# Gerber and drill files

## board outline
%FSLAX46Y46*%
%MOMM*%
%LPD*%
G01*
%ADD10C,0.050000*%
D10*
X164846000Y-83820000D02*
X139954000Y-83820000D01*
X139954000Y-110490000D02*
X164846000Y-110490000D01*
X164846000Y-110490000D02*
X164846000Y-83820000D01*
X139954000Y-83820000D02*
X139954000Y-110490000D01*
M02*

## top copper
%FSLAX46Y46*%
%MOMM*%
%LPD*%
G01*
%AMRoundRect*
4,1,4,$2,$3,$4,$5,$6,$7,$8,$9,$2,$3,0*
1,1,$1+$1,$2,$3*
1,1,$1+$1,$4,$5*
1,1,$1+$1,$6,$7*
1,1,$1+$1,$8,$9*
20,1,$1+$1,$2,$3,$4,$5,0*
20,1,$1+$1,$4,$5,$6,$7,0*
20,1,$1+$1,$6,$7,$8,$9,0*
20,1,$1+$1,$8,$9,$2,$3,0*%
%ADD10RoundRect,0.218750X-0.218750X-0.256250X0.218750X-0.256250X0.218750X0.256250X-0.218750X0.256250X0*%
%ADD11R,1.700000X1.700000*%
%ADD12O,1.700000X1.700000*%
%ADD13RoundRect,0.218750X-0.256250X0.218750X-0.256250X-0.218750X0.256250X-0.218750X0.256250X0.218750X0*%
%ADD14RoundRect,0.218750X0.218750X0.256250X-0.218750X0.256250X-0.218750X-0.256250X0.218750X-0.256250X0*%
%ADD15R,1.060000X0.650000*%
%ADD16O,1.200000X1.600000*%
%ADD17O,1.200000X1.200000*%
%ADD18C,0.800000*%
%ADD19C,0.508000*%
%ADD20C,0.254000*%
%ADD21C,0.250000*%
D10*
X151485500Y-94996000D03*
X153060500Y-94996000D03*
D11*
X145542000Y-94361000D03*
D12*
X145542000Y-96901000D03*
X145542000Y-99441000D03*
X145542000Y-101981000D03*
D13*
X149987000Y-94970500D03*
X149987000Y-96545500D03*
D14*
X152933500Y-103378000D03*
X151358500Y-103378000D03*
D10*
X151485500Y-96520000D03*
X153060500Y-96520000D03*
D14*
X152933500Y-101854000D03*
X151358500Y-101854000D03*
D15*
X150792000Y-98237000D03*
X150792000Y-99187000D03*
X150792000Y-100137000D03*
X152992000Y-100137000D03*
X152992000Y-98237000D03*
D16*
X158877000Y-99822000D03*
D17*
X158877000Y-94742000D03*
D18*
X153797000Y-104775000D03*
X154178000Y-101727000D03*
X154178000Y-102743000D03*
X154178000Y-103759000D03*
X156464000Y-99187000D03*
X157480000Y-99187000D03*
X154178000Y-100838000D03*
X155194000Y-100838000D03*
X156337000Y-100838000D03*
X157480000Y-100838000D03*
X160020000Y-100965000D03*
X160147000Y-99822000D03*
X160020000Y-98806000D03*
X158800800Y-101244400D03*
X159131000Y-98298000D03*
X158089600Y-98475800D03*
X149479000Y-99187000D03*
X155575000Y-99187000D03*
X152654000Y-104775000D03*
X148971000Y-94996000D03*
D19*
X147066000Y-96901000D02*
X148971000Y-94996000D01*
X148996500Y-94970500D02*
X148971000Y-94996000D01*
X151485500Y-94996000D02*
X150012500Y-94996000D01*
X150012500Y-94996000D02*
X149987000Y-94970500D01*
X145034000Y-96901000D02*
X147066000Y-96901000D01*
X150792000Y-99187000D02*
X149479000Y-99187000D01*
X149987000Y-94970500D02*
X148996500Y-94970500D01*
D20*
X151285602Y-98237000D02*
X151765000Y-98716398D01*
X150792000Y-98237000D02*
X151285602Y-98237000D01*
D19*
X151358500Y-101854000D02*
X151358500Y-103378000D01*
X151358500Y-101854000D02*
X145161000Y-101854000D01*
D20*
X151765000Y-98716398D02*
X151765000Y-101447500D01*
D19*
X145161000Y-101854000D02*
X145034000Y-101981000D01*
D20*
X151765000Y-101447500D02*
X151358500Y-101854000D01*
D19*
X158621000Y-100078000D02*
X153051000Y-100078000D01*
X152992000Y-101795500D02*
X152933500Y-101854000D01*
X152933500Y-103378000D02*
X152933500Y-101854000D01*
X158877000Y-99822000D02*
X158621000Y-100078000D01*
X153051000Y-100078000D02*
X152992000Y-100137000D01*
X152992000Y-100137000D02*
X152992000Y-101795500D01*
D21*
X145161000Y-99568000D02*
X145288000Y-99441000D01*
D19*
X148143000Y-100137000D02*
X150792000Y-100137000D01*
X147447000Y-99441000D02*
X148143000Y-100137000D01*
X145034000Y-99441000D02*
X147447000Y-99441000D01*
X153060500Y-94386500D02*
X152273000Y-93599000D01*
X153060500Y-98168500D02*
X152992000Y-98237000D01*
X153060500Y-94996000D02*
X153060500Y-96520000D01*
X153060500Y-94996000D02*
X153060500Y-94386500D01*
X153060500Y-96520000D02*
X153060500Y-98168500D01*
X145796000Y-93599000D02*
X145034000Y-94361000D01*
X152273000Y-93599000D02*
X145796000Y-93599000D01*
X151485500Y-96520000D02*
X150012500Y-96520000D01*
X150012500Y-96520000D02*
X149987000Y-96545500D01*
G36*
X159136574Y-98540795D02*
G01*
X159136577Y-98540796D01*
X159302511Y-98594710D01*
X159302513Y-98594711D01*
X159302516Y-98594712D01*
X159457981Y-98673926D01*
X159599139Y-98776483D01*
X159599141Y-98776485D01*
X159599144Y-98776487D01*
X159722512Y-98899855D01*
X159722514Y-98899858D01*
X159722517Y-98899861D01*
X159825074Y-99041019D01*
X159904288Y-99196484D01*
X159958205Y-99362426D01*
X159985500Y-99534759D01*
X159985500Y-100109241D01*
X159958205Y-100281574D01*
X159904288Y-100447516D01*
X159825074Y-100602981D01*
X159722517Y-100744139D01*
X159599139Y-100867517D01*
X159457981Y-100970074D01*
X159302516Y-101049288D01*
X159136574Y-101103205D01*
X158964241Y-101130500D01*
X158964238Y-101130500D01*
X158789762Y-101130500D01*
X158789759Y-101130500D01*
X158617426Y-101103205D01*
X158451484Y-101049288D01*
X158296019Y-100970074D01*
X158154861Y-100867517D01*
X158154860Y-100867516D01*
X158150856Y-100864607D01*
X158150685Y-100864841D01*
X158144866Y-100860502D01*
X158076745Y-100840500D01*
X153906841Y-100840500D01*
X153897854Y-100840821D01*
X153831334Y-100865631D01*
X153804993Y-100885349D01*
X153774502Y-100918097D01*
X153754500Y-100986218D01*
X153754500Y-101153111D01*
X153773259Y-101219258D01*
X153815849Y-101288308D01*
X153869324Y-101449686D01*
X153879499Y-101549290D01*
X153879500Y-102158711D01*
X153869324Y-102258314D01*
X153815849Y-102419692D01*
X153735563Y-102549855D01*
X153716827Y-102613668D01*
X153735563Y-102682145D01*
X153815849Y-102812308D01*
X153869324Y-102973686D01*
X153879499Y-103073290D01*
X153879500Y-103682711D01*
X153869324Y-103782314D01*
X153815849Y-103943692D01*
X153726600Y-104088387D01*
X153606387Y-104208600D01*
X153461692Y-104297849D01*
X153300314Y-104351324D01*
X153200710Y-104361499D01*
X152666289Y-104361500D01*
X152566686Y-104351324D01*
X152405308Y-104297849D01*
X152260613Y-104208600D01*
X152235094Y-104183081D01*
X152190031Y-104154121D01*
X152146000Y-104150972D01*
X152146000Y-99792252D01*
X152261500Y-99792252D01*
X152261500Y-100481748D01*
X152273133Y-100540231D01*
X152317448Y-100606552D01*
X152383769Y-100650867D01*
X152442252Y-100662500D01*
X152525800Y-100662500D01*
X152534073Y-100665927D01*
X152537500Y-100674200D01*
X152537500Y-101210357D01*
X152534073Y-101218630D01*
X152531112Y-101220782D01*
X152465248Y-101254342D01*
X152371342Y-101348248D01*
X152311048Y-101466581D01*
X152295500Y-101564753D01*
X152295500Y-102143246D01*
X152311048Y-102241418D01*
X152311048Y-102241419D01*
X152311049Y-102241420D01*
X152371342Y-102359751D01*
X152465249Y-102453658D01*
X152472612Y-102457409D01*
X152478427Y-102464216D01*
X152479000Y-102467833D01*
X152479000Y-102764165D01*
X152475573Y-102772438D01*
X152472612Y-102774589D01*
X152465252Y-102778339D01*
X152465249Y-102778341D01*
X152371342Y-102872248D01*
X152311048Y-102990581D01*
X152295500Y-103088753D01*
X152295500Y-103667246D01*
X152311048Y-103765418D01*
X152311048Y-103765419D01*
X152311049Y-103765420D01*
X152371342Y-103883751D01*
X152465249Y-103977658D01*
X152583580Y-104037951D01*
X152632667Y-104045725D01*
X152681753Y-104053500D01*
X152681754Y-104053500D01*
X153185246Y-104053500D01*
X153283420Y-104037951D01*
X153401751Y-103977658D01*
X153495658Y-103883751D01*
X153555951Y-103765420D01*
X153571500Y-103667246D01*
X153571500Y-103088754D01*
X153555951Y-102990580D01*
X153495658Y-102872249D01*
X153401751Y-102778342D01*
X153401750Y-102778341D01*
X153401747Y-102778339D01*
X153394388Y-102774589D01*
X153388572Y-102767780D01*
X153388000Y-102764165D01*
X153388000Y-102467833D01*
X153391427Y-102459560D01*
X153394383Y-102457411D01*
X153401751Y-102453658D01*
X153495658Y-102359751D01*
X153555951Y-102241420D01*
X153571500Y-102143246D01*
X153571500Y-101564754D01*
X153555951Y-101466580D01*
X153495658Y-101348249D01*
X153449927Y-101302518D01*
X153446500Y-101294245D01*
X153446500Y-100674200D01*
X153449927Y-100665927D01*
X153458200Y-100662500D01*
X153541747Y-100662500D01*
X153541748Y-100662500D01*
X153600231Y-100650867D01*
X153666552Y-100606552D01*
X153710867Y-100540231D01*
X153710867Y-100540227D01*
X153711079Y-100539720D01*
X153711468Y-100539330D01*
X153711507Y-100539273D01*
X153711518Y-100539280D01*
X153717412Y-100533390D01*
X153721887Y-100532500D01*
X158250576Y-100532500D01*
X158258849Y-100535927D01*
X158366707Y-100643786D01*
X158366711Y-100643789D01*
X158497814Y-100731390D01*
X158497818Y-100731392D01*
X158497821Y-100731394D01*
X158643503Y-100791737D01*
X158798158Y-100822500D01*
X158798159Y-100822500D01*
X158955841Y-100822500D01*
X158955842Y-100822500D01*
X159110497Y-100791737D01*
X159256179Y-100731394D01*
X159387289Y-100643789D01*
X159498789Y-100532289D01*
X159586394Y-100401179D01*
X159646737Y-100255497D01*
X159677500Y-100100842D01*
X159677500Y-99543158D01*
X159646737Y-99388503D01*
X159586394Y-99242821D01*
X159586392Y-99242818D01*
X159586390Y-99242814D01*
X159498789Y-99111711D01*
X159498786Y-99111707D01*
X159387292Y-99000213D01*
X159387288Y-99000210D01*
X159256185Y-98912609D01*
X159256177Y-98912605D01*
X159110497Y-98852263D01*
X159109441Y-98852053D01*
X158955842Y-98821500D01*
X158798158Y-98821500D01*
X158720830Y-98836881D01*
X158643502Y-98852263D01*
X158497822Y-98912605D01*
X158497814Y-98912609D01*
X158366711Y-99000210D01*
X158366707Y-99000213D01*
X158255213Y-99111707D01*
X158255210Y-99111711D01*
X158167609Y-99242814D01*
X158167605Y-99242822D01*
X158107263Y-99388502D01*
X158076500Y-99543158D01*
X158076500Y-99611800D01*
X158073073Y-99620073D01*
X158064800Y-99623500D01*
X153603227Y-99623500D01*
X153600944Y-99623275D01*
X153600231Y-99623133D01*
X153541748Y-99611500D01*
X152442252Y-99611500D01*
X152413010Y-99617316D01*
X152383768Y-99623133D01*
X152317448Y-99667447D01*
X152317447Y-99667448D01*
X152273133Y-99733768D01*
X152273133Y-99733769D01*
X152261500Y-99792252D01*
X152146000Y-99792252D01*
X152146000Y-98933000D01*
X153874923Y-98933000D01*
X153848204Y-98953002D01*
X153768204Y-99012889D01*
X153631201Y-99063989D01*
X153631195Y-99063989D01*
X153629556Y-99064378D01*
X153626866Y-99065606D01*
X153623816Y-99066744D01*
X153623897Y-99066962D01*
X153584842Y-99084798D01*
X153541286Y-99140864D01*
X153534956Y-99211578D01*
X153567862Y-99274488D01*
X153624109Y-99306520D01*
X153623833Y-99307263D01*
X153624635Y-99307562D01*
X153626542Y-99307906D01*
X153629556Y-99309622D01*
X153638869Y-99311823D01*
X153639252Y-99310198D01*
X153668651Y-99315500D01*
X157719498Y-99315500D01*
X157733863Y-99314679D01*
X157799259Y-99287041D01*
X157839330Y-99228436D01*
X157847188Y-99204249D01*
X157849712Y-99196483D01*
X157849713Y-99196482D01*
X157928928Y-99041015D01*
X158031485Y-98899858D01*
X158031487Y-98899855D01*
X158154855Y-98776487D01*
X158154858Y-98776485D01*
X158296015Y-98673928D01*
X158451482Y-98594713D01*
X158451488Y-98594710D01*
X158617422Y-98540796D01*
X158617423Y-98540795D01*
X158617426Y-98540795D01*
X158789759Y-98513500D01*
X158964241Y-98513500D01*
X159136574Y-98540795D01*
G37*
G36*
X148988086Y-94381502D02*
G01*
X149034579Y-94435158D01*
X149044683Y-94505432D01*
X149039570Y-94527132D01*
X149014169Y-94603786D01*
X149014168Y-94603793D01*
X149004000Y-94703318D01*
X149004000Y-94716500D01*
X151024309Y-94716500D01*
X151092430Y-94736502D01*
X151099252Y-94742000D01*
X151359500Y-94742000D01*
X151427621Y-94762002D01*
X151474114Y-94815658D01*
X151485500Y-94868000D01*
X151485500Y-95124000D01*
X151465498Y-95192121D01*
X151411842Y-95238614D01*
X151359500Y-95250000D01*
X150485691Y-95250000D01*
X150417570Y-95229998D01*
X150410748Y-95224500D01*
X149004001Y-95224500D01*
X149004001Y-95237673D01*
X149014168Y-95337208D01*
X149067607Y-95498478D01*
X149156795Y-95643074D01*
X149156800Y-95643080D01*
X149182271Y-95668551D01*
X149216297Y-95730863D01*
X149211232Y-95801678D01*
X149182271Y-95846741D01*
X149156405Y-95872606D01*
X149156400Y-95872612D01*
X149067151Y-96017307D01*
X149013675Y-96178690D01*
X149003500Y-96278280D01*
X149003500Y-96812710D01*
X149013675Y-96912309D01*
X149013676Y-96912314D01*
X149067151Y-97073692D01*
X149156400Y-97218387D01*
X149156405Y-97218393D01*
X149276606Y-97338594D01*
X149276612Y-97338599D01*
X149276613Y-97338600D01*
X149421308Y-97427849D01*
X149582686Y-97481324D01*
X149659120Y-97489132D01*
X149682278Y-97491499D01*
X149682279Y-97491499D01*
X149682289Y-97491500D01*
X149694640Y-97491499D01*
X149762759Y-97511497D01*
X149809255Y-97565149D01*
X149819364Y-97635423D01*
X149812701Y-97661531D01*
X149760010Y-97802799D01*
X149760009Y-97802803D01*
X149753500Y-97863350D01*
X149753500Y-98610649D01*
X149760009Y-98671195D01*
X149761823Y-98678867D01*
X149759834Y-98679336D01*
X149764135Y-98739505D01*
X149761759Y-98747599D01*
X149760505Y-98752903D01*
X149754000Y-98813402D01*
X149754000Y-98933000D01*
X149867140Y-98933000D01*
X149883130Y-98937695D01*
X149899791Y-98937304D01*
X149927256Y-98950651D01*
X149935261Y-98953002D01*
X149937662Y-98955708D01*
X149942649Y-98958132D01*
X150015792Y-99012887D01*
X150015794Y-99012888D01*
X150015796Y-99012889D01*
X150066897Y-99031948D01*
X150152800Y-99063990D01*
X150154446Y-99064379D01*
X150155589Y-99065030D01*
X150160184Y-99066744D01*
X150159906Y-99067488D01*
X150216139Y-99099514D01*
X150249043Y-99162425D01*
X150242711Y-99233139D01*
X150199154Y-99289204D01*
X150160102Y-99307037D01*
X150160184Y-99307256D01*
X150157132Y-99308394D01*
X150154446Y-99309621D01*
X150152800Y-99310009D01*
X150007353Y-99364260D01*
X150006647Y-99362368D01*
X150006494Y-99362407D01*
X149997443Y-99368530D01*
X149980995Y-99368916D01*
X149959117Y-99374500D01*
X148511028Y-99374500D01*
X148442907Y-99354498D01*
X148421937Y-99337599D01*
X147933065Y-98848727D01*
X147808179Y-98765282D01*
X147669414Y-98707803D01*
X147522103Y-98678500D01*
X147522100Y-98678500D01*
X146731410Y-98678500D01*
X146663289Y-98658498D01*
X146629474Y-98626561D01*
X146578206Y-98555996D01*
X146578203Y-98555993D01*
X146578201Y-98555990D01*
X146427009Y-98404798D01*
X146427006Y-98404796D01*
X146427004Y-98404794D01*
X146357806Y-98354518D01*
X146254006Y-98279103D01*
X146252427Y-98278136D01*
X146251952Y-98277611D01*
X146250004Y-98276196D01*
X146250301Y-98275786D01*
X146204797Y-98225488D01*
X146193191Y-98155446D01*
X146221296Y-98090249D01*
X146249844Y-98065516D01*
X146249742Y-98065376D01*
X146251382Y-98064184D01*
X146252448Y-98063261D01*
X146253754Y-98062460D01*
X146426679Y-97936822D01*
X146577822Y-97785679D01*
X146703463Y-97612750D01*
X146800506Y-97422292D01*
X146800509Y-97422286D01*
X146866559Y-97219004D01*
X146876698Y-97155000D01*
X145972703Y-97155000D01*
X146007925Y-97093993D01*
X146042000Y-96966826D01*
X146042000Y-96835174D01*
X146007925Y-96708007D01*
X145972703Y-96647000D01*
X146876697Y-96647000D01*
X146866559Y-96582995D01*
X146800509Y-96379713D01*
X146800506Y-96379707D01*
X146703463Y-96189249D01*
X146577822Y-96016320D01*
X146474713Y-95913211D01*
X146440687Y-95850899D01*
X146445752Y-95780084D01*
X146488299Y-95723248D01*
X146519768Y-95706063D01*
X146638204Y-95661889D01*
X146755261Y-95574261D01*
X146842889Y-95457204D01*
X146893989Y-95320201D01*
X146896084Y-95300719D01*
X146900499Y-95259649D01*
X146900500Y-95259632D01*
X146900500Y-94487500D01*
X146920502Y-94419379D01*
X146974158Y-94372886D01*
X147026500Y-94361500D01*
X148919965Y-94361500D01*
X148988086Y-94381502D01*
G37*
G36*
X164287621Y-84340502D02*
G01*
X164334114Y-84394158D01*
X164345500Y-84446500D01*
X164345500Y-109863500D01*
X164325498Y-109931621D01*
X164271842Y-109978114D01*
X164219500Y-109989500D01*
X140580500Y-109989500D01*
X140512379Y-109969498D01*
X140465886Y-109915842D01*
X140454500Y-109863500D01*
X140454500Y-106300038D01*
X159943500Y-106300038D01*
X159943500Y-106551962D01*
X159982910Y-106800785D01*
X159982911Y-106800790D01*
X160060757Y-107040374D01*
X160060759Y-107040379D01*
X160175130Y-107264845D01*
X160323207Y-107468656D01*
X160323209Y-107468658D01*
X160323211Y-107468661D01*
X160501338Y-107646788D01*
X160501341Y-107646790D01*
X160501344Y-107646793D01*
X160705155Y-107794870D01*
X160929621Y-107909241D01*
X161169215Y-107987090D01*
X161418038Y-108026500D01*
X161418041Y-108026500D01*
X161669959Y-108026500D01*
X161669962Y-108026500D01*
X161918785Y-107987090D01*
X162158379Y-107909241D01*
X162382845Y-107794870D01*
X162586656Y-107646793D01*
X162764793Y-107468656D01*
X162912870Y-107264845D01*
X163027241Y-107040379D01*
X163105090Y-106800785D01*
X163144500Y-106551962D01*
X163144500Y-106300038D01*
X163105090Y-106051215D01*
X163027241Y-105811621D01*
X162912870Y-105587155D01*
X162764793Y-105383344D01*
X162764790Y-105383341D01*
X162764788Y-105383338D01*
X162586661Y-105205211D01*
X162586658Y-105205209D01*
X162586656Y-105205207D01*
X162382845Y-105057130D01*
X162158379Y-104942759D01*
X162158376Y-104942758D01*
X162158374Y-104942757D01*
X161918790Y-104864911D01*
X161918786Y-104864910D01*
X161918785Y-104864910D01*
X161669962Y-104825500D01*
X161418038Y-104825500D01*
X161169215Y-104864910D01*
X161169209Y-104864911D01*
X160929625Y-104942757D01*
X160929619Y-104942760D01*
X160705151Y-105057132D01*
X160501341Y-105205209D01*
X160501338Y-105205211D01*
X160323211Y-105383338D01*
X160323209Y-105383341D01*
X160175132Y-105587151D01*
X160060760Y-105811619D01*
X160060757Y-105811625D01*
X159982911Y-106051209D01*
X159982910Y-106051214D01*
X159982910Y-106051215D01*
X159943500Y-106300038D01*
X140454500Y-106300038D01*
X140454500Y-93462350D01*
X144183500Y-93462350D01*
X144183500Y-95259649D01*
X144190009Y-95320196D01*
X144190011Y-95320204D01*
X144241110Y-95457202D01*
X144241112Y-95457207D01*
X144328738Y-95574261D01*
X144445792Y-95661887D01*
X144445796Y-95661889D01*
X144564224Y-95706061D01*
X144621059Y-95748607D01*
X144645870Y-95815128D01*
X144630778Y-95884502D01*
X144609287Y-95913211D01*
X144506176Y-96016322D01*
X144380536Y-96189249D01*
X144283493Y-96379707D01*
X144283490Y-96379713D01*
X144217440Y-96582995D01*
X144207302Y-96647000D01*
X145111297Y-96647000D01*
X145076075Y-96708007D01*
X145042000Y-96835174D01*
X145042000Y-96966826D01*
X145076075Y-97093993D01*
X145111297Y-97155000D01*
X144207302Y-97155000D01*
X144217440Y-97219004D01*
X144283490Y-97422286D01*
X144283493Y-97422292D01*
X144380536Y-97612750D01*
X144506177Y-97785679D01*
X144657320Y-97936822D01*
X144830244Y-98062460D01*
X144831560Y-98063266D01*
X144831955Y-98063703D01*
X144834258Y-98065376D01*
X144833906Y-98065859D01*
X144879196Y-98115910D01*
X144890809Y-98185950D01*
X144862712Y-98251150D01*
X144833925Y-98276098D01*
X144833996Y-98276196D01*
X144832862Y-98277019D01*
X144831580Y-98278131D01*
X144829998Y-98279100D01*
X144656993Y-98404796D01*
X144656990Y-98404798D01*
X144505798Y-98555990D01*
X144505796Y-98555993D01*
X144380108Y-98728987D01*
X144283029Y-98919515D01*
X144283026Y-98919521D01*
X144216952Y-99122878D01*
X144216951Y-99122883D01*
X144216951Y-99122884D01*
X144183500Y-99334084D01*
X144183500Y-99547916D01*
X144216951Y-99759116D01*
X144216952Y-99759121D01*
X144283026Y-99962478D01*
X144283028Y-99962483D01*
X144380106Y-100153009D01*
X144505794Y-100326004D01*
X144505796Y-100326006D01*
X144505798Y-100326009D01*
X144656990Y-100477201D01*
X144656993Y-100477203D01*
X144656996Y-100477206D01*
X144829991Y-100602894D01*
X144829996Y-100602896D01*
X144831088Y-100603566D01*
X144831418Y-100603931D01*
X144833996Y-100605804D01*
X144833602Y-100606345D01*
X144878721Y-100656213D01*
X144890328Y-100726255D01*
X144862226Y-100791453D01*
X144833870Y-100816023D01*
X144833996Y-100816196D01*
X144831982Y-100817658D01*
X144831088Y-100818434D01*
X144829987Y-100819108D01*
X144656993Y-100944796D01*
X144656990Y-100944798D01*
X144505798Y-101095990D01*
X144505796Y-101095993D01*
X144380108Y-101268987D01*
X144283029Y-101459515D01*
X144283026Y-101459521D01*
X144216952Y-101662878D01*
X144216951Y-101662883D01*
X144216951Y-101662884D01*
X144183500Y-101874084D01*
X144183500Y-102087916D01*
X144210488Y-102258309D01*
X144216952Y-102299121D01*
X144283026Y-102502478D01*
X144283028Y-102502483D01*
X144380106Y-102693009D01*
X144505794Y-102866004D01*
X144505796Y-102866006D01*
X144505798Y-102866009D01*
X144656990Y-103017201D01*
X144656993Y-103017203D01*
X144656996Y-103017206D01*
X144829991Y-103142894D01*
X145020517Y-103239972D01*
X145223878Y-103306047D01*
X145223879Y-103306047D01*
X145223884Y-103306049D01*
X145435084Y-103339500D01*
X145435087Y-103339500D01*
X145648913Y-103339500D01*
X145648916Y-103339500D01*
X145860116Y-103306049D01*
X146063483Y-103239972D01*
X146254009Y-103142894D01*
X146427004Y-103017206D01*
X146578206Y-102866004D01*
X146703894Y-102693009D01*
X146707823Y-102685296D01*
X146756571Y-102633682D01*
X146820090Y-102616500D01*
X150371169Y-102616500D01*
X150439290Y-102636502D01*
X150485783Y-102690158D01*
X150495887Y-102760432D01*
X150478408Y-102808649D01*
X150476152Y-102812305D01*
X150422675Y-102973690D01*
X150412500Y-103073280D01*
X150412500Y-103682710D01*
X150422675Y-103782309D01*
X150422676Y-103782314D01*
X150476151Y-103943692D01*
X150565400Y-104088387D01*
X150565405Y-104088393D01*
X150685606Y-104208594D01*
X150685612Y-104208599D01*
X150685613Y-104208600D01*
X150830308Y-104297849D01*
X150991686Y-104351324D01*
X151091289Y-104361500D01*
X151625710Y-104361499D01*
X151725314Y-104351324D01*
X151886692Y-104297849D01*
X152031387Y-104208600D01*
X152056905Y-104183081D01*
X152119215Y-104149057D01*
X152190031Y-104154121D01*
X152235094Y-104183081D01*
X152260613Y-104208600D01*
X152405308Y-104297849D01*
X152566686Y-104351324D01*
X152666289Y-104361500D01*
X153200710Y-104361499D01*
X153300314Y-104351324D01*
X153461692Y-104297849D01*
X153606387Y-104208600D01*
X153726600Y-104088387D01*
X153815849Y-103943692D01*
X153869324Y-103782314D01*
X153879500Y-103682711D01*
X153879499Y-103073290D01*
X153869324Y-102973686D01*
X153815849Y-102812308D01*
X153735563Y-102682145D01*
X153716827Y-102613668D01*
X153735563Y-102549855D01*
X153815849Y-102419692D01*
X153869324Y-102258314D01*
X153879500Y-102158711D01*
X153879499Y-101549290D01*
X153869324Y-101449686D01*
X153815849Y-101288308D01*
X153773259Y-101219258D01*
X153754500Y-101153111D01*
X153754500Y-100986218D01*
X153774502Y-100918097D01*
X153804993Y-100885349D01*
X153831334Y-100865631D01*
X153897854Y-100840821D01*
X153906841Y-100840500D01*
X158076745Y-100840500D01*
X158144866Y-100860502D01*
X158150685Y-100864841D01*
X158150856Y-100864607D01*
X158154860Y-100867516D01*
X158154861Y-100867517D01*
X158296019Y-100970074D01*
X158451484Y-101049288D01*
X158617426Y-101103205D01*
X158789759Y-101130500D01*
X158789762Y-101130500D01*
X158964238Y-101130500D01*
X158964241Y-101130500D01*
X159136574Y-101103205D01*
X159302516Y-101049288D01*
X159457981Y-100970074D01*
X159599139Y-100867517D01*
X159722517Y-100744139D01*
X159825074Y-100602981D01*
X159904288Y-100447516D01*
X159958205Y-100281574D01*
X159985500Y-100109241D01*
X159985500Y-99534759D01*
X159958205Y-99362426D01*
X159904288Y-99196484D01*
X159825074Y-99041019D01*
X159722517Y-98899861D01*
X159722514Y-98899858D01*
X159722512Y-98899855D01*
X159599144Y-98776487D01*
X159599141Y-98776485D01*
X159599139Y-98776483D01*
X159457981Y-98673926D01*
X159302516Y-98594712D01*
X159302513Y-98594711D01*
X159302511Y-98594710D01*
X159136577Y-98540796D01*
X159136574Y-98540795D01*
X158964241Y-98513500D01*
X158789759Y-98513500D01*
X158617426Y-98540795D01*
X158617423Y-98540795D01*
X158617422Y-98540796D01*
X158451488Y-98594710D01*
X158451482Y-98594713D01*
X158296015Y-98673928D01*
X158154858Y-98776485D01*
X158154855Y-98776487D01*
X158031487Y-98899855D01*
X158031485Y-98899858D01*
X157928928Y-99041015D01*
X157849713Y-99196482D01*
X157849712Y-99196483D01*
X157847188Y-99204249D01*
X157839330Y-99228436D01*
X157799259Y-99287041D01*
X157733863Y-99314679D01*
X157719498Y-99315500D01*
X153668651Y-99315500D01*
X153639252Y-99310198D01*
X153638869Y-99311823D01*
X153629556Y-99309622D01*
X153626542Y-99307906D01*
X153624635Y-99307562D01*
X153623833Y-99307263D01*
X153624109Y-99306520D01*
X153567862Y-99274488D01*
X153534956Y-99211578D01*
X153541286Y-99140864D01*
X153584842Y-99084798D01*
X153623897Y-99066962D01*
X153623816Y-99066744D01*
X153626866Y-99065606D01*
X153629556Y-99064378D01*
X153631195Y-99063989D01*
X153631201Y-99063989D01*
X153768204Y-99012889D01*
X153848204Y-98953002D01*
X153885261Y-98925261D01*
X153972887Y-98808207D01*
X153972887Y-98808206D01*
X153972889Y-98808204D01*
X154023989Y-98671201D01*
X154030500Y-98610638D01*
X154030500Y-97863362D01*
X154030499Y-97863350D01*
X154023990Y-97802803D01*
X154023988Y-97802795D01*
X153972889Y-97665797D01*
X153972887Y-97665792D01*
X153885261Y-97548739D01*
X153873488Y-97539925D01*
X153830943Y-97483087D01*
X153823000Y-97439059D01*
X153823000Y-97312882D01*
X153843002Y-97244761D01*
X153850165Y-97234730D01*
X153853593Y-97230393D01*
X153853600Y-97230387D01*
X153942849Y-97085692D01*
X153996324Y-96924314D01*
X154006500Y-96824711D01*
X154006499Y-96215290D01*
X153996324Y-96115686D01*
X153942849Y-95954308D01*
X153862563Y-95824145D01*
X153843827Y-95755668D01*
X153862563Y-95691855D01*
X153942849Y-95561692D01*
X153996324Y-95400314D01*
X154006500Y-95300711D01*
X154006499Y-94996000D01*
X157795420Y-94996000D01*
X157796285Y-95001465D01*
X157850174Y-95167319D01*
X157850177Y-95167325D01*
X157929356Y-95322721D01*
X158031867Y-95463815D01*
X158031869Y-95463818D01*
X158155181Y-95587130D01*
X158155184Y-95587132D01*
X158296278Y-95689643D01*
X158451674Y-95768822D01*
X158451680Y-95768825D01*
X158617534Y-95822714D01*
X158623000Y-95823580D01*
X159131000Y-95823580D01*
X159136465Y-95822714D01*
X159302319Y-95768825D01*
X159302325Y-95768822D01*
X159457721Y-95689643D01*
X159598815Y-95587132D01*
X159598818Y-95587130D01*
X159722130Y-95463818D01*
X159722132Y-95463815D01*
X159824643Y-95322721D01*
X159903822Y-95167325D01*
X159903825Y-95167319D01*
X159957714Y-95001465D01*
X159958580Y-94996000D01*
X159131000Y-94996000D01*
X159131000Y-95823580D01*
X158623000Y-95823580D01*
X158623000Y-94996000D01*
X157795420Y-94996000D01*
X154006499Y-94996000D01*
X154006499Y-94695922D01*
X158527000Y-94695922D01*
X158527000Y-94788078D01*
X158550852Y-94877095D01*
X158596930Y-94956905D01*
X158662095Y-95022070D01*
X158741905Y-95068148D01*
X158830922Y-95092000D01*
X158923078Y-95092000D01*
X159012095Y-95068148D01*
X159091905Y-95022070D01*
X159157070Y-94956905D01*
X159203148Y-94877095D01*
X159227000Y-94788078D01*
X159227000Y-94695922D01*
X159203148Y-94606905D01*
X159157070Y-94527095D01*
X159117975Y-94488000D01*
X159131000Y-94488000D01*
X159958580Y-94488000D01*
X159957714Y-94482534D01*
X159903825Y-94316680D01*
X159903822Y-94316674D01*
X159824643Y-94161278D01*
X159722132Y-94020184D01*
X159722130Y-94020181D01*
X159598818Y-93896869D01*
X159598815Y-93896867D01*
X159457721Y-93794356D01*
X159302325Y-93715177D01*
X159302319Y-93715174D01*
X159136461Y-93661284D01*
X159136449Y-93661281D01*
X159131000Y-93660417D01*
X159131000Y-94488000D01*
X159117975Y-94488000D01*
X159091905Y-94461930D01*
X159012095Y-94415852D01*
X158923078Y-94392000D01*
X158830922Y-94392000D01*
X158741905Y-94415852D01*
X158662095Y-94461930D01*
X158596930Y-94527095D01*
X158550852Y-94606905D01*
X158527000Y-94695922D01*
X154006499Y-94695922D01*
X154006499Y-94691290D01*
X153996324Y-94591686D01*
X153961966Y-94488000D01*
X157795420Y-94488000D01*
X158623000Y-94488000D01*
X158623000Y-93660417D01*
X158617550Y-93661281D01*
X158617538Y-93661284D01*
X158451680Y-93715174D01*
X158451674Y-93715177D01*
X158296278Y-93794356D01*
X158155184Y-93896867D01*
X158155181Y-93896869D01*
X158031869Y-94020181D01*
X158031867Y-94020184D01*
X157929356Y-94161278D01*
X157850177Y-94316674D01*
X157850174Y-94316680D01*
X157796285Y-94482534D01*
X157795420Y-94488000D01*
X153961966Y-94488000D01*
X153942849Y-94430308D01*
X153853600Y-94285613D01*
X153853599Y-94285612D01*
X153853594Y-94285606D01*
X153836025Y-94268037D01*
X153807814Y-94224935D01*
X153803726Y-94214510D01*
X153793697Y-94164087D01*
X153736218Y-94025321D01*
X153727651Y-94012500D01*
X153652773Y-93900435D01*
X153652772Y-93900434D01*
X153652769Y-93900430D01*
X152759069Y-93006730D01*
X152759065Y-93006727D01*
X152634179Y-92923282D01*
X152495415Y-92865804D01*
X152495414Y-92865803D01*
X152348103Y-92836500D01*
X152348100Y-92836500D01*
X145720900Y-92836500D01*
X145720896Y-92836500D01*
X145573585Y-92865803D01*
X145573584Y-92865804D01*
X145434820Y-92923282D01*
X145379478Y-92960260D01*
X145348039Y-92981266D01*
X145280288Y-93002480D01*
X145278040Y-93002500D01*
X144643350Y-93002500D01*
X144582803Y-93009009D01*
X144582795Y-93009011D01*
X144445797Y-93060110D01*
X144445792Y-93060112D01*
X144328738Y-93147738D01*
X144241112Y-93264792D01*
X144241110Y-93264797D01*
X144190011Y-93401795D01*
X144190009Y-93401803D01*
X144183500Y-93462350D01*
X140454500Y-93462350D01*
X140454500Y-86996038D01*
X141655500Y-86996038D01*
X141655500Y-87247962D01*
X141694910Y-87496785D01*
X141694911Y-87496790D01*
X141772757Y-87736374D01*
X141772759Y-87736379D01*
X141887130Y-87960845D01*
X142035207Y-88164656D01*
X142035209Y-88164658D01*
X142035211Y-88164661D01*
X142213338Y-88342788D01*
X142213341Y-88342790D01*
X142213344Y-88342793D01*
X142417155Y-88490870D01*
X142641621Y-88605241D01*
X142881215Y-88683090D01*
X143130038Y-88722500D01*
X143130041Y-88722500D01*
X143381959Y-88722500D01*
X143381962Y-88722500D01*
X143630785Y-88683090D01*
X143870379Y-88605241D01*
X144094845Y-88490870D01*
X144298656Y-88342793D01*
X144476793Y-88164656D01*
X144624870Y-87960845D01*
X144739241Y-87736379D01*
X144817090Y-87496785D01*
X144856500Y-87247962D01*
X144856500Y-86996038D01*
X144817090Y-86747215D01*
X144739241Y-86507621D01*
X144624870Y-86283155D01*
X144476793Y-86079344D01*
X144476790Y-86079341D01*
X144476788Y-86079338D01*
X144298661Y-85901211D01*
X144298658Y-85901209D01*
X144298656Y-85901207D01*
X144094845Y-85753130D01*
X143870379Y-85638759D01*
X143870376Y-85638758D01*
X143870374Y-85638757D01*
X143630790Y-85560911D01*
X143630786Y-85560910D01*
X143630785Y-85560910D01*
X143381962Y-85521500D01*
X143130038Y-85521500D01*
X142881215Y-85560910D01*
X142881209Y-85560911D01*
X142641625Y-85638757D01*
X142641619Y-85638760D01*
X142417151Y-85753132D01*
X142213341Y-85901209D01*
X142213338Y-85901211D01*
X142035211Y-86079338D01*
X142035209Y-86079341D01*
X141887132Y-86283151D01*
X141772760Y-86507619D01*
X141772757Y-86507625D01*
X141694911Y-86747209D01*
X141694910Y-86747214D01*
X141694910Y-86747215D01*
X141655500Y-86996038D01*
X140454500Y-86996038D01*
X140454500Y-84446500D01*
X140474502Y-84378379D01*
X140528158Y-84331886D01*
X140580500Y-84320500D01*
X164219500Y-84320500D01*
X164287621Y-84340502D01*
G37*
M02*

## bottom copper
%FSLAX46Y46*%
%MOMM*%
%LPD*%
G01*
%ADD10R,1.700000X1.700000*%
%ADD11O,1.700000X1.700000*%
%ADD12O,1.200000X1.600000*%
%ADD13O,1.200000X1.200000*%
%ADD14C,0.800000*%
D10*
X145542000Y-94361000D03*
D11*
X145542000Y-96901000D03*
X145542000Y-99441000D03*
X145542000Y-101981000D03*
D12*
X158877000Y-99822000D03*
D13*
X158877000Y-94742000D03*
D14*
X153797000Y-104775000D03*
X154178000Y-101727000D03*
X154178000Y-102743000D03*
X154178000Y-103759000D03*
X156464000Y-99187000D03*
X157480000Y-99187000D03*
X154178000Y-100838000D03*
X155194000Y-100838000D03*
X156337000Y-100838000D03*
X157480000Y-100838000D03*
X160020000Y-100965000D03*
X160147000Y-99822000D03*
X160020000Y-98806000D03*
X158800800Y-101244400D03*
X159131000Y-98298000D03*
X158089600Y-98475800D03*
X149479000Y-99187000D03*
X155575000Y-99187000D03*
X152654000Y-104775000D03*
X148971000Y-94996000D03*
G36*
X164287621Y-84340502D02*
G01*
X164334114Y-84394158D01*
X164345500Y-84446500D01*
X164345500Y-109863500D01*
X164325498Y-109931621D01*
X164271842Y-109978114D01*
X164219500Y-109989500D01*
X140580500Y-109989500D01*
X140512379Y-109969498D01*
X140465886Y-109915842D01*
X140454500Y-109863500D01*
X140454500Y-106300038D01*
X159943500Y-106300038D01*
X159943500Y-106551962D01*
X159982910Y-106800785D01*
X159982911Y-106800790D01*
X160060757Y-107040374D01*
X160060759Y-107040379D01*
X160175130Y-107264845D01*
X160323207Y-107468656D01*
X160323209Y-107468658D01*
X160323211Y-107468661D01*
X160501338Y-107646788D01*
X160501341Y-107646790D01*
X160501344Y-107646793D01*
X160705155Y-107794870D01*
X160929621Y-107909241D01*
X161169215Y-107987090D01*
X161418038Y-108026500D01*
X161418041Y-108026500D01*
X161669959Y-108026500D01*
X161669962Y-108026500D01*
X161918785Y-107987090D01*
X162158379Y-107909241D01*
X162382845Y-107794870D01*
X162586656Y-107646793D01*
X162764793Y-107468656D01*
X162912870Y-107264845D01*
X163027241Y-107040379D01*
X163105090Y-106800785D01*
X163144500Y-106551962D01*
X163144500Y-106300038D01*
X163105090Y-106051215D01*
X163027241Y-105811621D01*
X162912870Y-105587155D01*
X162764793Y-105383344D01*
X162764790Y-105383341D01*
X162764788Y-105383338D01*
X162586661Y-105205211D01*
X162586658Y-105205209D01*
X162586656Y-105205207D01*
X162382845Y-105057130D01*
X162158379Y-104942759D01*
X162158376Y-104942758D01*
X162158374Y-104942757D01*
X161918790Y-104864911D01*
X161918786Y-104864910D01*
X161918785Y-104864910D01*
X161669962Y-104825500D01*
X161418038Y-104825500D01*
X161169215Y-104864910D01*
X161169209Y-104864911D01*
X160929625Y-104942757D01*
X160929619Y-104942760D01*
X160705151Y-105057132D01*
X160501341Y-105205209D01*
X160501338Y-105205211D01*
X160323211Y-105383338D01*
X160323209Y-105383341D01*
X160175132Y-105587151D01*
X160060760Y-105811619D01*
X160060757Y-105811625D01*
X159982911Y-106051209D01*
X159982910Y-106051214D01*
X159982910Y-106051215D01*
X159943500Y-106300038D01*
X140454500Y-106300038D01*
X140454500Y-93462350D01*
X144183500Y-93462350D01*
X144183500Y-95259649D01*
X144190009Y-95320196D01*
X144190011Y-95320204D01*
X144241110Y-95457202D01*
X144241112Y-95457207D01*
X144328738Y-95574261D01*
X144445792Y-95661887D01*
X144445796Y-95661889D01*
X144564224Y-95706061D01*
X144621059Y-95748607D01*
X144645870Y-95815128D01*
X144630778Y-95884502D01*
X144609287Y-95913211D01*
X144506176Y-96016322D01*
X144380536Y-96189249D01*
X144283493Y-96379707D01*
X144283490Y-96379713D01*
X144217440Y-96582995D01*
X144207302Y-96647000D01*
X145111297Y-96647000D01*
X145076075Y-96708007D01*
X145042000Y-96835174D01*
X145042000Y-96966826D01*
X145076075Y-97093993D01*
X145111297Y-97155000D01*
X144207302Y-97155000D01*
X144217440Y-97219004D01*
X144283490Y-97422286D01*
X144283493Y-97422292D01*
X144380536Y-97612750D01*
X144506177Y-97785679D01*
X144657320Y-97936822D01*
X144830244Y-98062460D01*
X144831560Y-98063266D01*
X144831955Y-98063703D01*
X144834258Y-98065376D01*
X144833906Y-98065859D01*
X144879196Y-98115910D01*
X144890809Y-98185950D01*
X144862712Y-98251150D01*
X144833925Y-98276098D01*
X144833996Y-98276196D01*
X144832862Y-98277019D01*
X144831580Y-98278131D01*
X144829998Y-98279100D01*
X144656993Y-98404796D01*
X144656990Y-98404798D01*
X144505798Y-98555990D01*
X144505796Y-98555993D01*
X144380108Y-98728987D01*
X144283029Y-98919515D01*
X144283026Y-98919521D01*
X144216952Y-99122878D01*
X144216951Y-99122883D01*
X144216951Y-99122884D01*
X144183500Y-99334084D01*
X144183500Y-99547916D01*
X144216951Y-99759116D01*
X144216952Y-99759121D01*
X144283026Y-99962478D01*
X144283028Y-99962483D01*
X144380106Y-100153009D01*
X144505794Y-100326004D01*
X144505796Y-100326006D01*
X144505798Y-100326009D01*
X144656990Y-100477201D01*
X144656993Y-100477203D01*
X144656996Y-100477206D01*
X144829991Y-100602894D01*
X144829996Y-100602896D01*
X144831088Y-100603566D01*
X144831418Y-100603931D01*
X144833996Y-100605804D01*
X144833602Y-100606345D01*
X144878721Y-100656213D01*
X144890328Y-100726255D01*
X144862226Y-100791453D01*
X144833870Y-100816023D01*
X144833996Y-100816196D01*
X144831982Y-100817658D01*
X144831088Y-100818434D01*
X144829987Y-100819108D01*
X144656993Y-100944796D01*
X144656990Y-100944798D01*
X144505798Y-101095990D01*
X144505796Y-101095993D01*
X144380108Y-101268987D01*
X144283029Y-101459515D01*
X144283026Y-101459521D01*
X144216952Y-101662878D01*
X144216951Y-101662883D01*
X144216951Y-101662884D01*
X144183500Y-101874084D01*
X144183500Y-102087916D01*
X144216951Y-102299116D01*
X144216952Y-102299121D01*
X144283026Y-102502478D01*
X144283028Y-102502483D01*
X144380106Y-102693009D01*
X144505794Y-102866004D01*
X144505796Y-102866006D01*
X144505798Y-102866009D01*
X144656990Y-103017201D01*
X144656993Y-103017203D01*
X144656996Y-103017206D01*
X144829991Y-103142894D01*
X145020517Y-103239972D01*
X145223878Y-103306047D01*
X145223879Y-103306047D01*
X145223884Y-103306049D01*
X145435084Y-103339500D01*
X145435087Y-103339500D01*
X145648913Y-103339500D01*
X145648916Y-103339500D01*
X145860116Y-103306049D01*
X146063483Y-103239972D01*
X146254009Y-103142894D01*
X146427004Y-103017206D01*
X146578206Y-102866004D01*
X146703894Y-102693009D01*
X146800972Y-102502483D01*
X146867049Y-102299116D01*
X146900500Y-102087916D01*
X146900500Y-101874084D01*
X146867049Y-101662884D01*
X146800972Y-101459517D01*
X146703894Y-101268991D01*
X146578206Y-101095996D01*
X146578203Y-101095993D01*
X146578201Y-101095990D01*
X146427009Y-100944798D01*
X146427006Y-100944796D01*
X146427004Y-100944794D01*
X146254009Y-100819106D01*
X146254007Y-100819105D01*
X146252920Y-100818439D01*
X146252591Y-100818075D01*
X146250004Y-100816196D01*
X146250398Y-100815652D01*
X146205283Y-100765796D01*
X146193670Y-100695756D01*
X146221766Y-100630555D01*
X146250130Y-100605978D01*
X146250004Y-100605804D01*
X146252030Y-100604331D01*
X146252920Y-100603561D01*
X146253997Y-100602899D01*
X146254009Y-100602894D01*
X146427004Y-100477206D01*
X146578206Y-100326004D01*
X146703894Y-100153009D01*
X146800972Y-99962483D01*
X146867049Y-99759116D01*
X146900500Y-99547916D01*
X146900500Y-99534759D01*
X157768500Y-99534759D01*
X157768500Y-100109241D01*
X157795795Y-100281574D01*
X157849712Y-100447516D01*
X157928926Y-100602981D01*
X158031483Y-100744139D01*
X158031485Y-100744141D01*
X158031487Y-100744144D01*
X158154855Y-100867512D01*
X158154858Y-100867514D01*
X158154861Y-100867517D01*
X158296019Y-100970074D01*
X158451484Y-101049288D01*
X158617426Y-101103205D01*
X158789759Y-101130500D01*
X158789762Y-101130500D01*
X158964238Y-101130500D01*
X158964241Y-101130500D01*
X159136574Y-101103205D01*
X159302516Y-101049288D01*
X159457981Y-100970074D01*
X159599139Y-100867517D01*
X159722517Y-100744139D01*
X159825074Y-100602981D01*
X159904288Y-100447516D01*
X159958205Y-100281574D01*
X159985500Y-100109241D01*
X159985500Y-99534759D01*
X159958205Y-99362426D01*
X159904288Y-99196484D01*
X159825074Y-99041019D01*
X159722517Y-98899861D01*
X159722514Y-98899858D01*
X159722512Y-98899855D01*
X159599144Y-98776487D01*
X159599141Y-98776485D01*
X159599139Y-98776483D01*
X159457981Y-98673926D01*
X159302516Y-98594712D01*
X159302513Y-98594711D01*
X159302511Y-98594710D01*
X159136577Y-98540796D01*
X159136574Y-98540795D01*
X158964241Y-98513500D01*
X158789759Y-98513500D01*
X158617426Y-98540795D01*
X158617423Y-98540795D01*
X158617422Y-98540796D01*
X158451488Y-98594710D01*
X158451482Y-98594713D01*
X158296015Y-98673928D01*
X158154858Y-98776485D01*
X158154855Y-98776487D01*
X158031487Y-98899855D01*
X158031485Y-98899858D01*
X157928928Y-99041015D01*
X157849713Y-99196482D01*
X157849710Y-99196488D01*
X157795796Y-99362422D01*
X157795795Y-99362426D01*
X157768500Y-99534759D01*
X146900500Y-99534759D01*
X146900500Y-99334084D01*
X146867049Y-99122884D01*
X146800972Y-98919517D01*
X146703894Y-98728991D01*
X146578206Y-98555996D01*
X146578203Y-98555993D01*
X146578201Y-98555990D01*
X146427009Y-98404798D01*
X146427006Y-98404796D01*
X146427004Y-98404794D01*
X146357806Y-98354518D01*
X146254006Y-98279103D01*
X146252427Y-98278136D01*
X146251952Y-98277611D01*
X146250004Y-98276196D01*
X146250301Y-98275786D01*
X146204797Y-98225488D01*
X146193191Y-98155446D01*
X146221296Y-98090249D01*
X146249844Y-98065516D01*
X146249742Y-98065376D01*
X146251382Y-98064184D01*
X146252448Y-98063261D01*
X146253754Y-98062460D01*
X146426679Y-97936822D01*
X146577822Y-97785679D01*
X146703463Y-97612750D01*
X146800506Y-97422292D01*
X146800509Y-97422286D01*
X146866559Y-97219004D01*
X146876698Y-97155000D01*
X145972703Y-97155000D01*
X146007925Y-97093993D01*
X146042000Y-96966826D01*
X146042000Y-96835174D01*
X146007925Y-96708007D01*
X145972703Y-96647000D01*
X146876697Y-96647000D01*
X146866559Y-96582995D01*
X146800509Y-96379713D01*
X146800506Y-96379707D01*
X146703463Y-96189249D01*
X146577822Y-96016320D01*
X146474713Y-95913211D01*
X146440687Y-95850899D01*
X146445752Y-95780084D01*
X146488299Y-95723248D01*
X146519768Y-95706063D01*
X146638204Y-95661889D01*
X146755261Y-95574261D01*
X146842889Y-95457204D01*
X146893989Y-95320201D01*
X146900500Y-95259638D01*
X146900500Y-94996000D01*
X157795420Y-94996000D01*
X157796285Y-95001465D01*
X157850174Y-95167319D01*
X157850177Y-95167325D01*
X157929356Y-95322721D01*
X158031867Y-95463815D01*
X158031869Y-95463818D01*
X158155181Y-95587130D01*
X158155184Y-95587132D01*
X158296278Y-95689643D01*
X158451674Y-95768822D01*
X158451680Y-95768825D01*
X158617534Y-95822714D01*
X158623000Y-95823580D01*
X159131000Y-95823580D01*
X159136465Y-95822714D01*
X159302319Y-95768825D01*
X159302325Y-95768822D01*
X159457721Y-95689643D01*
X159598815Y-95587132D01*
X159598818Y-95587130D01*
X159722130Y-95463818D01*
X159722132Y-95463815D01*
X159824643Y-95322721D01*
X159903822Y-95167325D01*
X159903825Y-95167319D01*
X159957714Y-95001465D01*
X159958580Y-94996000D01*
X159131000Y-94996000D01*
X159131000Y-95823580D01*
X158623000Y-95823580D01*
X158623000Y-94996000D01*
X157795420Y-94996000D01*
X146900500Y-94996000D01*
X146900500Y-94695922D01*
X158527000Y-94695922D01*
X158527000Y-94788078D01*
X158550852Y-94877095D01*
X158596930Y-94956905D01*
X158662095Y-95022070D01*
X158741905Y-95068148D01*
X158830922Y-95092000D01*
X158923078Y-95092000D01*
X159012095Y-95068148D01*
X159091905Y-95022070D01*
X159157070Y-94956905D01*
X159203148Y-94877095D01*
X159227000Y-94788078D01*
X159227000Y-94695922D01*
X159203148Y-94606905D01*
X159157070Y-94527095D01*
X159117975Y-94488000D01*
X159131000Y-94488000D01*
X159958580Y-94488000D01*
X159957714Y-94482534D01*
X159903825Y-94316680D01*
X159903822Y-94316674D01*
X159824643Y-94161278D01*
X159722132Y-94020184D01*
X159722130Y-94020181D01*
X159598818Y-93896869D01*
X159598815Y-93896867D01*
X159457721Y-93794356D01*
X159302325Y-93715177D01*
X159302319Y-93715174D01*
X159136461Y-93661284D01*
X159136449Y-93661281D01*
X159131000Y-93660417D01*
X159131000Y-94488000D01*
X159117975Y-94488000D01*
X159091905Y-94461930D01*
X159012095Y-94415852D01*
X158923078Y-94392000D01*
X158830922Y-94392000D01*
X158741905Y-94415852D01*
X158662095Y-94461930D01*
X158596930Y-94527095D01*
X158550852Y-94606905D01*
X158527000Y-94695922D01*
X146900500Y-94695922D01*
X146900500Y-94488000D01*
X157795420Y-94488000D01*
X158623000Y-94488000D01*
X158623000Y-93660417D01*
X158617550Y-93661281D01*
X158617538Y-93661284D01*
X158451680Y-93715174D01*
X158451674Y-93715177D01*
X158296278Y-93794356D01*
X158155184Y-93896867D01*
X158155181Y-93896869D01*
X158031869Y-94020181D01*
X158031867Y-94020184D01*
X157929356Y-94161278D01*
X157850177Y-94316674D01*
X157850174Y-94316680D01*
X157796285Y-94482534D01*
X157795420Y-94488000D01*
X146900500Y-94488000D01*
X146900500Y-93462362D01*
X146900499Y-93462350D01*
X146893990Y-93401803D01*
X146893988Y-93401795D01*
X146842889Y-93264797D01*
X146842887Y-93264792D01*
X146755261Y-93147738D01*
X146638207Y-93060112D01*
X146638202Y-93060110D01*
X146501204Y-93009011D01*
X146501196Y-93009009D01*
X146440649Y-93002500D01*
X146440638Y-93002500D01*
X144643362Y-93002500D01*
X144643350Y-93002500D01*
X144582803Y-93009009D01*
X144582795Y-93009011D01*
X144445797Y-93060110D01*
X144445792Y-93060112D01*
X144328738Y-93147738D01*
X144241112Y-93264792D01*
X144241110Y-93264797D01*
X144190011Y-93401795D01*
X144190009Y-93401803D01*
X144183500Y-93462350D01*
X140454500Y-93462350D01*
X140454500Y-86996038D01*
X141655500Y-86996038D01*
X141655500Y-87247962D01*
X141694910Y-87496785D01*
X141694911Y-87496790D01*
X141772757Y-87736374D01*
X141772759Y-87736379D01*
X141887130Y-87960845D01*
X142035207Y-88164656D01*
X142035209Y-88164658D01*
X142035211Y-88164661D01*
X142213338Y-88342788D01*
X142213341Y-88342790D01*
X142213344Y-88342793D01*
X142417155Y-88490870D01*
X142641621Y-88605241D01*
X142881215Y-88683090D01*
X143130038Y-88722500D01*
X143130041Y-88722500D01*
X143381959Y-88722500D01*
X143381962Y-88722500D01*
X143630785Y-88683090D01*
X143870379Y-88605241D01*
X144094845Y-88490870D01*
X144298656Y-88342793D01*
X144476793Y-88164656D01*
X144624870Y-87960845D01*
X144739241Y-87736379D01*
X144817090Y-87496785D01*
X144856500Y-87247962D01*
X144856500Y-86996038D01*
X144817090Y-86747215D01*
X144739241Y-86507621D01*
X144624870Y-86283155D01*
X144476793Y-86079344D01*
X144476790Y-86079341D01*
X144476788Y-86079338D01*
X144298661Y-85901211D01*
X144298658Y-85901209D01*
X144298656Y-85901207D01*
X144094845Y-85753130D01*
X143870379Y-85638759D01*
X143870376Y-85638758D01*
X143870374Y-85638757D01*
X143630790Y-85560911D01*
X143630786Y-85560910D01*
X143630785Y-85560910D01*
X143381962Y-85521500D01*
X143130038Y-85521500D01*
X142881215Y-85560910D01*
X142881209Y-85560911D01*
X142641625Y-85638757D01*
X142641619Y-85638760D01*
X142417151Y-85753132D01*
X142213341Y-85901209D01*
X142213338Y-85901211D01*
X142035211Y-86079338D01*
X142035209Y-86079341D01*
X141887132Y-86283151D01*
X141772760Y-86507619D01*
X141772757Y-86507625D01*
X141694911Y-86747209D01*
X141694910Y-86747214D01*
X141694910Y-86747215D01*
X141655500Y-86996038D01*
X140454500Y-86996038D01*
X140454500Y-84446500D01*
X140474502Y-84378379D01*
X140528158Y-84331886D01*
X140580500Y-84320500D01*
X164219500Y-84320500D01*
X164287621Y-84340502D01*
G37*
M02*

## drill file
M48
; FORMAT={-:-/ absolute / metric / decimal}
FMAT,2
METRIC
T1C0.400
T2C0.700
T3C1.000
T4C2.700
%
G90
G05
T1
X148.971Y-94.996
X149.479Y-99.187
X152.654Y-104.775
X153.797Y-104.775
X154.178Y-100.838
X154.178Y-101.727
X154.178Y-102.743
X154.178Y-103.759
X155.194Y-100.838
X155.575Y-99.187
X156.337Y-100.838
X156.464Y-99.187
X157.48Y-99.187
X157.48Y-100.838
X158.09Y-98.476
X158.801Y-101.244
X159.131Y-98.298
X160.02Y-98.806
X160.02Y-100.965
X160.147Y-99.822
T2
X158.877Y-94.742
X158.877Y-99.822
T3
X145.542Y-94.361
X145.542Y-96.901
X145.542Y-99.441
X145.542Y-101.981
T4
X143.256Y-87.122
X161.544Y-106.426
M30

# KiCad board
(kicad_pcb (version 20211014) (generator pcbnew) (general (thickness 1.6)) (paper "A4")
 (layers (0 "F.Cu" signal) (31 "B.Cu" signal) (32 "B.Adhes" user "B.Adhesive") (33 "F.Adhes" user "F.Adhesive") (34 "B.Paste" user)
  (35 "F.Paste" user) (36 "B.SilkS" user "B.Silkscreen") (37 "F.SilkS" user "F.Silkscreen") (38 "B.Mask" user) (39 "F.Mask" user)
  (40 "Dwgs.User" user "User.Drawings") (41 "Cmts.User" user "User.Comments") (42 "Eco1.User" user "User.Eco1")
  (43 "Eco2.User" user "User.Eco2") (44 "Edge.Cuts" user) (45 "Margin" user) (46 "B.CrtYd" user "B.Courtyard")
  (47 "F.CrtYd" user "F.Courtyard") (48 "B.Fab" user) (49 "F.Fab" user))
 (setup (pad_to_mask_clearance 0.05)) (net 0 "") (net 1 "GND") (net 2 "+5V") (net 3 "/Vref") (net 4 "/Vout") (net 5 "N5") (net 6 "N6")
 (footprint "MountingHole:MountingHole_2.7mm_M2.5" (layer "F.Cu") (at 161.544 106.426)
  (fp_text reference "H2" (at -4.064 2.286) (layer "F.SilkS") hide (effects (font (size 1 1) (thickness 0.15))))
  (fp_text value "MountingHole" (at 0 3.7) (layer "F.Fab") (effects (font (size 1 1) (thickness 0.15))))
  (pad "" np_thru_hole circle locked (at 0 0) (size 2.7 2.7) (drill 2.7) (layers *.Cu *.Mask)))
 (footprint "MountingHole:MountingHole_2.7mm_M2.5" (layer "F.Cu") (at 143.256 87.122)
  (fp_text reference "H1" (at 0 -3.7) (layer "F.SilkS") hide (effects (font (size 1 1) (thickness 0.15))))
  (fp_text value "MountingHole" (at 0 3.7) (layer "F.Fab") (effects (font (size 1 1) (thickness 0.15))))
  (pad "" np_thru_hole circle locked (at 0 0) (size 2.7 2.7) (drill 2.7) (layers *.Cu *.Mask)))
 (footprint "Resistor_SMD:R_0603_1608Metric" (layer "F.Cu") (at 152.273 94.996)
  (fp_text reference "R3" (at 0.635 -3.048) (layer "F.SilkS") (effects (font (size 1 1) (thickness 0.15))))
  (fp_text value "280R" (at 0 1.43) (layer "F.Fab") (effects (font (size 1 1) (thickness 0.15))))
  (pad "1" smd roundrect locked (at -0.7875 0) (size 0.875 0.95) (layers "F.Cu" "F.Paste" "F.Mask") (roundrect_rratio 0.25) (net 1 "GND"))
  (pad "2" smd roundrect locked (at 0.7875 0) (size 0.875 0.95) (layers "F.Cu" "F.Paste" "F.Mask") (roundrect_rratio 0.25) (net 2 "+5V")))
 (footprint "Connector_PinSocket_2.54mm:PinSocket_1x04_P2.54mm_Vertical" (layer "F.Cu") (at 145.542 94.361)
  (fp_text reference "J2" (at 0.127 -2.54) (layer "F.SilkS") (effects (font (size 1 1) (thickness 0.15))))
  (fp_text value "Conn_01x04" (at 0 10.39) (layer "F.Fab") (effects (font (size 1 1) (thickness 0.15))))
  (pad "1" thru_hole rect locked (at 0 0) (size 1.7 1.7) (drill 1) (layers *.Cu *.Mask) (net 2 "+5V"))
  (pad "2" thru_hole oval locked (at 0 2.54) (size 1.7 1.7) (drill 1) (layers *.Cu *.Mask) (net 1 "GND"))
  (pad "3" thru_hole oval locked (at 0 5.08) (size 1.7 1.7) (drill 1) (layers *.Cu *.Mask) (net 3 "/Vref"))
  (pad "4" thru_hole oval locked (at 0 7.62) (size 1.7 1.7) (drill 1) (layers *.Cu *.Mask) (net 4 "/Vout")))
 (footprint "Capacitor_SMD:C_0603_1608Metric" (layer "F.Cu") (at 149.987 95.758 -90)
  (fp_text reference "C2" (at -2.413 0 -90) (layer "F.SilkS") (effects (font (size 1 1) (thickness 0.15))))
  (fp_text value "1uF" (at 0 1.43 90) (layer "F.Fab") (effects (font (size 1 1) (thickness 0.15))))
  (pad "1" smd roundrect locked (at -0.7875 0 270) (size 0.875 0.95) (layers "F.Cu" "F.Paste" "F.Mask") (roundrect_rratio 0.25)
   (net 1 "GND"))
  (pad "2" smd roundrect locked (at 0.7875 0 270) (size 0.875 0.95) (layers "F.Cu" "F.Paste" "F.Mask") (roundrect_rratio 0.25) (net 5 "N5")))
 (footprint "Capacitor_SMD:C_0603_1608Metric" (layer "F.Cu") (at 152.146 103.378 180)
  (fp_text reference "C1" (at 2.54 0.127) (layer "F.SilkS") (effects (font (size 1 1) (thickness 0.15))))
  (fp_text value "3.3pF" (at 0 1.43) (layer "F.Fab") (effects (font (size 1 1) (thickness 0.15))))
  (pad "1" smd roundrect locked (at -0.7875 0 180) (size 0.875 0.95) (layers "F.Cu" "F.Paste" "F.Mask") (roundrect_rratio 0.25) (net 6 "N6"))
  (pad "2" smd roundrect locked (at 0.7875 0 180) (size 0.875 0.95) (layers "F.Cu" "F.Paste" "F.Mask") (roundrect_rratio 0.25)
   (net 4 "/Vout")))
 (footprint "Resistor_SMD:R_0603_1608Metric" (layer "F.Cu") (at 152.273 96.52)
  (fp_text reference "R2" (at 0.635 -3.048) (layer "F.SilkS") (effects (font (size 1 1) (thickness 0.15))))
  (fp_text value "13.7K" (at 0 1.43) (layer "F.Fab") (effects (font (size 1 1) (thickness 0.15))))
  (pad "1" smd roundrect locked (at -0.7875 0) (size 0.875 0.95) (layers "F.Cu" "F.Paste" "F.Mask") (roundrect_rratio 0.25) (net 5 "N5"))
  (pad "2" smd roundrect locked (at 0.7875 0) (size 0.875 0.95) (layers "F.Cu" "F.Paste" "F.Mask") (roundrect_rratio 0.25) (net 2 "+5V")))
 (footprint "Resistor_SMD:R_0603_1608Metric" (layer "F.Cu") (at 152.146 101.854 180)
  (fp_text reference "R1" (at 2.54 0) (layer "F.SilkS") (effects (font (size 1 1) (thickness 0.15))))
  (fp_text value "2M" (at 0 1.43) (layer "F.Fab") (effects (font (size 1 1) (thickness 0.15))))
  (pad "1" smd roundrect locked (at -0.7875 0 180) (size 0.875 0.95) (layers "F.Cu" "F.Paste" "F.Mask") (roundrect_rratio 0.25) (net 6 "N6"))
  (pad "2" smd roundrect locked (at 0.7875 0 180) (size 0.875 0.95) (layers "F.Cu" "F.Paste" "F.Mask") (roundrect_rratio 0.25)
   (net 4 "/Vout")))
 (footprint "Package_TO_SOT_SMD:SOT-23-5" (layer "F.Cu") (at 151.892 99.187)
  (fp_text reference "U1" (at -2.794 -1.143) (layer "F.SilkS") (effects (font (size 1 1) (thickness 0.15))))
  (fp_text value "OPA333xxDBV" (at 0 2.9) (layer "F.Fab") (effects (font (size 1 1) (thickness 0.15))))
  (pad "1" smd rect locked (at -1.1 -0.95) (size 1.06 0.65) (layers "F.Cu" "F.Paste" "F.Mask") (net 4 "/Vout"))
  (pad "2" smd rect locked (at -1.1 0) (size 1.06 0.65) (layers "F.Cu" "F.Paste" "F.Mask") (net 1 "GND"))
  (pad "3" smd rect locked (at -1.1 0.95) (size 1.06 0.65) (layers "F.Cu" "F.Paste" "F.Mask") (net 3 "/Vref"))
  (pad "4" smd rect locked (at 1.1 0.95) (size 1.06 0.65) (layers "F.Cu" "F.Paste" "F.Mask") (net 6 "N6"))
  (pad "5" smd rect locked (at 1.1 -0.95) (size 1.06 0.65) (layers "F.Cu" "F.Paste" "F.Mask") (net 2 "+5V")))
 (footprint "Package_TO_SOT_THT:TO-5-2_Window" (layer "F.Cu") (at 158.877 99.822 90)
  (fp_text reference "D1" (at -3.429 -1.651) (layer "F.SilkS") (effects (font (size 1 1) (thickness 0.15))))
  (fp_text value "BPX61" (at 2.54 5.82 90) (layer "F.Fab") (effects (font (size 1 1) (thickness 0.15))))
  (pad "1" thru_hole oval locked (at 0 0 90) (size 1.6 1.2) (drill 0.7) (layers *.Cu *.Mask) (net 6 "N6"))
  (pad "2" thru_hole oval locked (at 5.08 0 90) (size 1.2 1.2) (drill 0.7) (layers *.Cu *.Mask) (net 1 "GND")))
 (gr_line (start 164.846 83.82) (end 139.954 83.82) (layer "Edge.Cuts") (width 0.05))
 (gr_line (start 139.954 110.49) (end 164.846 110.49) (layer "Edge.Cuts") (width 0.05))
 (gr_line (start 164.846 110.49) (end 164.846 83.82) (layer "Edge.Cuts") (width 0.05))
 (gr_line (start 139.954 83.82) (end 139.954 110.49) (layer "Edge.Cuts") (width 0.05))
 (segment (start 147.066 96.901) (end 148.971 94.996) (width 0.508) (layer "F.Cu") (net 1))
 (segment (start 148.9965 94.9705) (end 148.971 94.996) (width 0.508) (layer "F.Cu") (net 1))
 (segment (start 151.4855 94.996) (end 150.0125 94.996) (width 0.508) (layer "F.Cu") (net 1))
 (segment (start 150.0125 94.996) (end 149.987 94.9705) (width 0.508) (layer "F.Cu") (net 1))
 (segment (start 145.034 96.901) (end 147.066 96.901) (width 0.508) (layer "F.Cu") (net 1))
 (segment (start 150.792 99.187) (end 149.479 99.187) (width 0.508) (layer "F.Cu") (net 1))
 (segment (start 149.987 94.9705) (end 148.9965 94.9705) (width 0.508) (layer "F.Cu") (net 1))
 (via (at 153.797 104.775) (size 0.8) (drill 0.4) (layers "F.Cu" "B.Cu") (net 1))
 (via (at 154.178 101.727) (size 0.8) (drill 0.4) (layers "F.Cu" "B.Cu") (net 1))
 (via (at 154.178 102.743) (size 0.8) (drill 0.4) (layers "F.Cu" "B.Cu") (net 1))
 (via (at 154.178 103.759) (size 0.8) (drill 0.4) (layers "F.Cu" "B.Cu") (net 1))
 (via (at 156.464 99.187) (size 0.8) (drill 0.4) (layers "F.Cu" "B.Cu") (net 1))
 (via (at 157.48 99.187) (size 0.8) (drill 0.4) (layers "F.Cu" "B.Cu") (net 1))
 (via (at 154.178 100.838) (size 0.8) (drill 0.4) (layers "F.Cu" "B.Cu") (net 1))
 (via (at 155.194 100.838) (size 0.8) (drill 0.4) (layers "F.Cu" "B.Cu") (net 1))
 (via (at 156.337 100.838) (size 0.8) (drill 0.4) (layers "F.Cu" "B.Cu") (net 1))
 (via (at 157.48 100.838) (size 0.8) (drill 0.4) (layers "F.Cu" "B.Cu") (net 1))
 (via (at 160.02 100.965) (size 0.8) (drill 0.4) (layers "F.Cu" "B.Cu") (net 1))
 (via (at 160.147 99.822) (size 0.8) (drill 0.4) (layers "F.Cu" "B.Cu") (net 1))
 (via (at 160.02 98.806) (size 0.8) (drill 0.4) (layers "F.Cu" "B.Cu") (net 1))
 (via (at 158.8008 101.2444) (size 0.8) (drill 0.4) (layers "F.Cu" "B.Cu") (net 1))
 (via (at 159.131 98.298) (size 0.8) (drill 0.4) (layers "F.Cu" "B.Cu") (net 1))
 (via (at 158.0896 98.4758) (size 0.8) (drill 0.4) (layers "F.Cu" "B.Cu") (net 1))
 (via (at 149.479 99.187) (size 0.8) (drill 0.4) (layers "F.Cu" "B.Cu") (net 1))
 (via (at 155.575 99.187) (size 0.8) (drill 0.4) (layers "F.Cu" "B.Cu") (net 1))
 (via (at 152.654 104.775) (size 0.8) (drill 0.4) (layers "F.Cu" "B.Cu") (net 1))
 (via (at 148.971 94.996) (size 0.8) (drill 0.4) (layers "F.Cu" "B.Cu") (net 1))
 (segment (start 151.285602 98.237) (end 151.765 98.716398) (width 0.254) (layer "F.Cu") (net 4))
 (segment (start 150.792 98.237) (end 151.285602 98.237) (width 0.254) (layer "F.Cu") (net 4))
 (segment (start 151.3585 101.854) (end 151.3585 103.378) (width 0.508) (layer "F.Cu") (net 4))
 (segment (start 151.3585 101.854) (end 145.161 101.854) (width 0.508) (layer "F.Cu") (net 4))
 (segment (start 151.765 98.716398) (end 151.765 101.4475) (width 0.254) (layer "F.Cu") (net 4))
 (segment (start 145.161 101.854) (end 145.034 101.981) (width 0.508) (layer "F.Cu") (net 4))
 (segment (start 151.765 101.4475) (end 151.3585 101.854) (width 0.254) (layer "F.Cu") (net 4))
 (segment (start 158.621 100.078) (end 153.051 100.078) (width 0.508) (layer "F.Cu") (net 6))
 (segment (start 152.992 101.7955) (end 152.9335 101.854) (width 0.508) (layer "F.Cu") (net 6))
 (segment (start 152.9335 103.378) (end 152.9335 101.854) (width 0.508) (layer "F.Cu") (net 6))
 (segment (start 158.877 99.822) (end 158.621 100.078) (width 0.508) (layer "F.Cu") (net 6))
 (segment (start 153.051 100.078) (end 152.992 100.137) (width 0.508) (layer "F.Cu") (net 6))
 (segment (start 152.992 100.137) (end 152.992 101.7955) (width 0.508) (layer "F.Cu") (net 6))
 (segment (start 145.161 99.568) (end 145.288 99.441) (width 0.25) (layer "F.Cu") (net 3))
 (segment (start 148.143 100.137) (end 150.792 100.137) (width 0.508) (layer "F.Cu") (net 3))
 (segment (start 147.447 99.441) (end 148.143 100.137) (width 0.508) (layer "F.Cu") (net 3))
 (segment (start 145.034 99.441) (end 147.447 99.441) (width 0.508) (layer "F.Cu") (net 3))
 (segment (start 153.0605 94.3865) (end 152.273 93.599) (width 0.508) (layer "F.Cu") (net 2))
 (segment (start 153.0605 98.1685) (end 152.992 98.237) (width 0.508) (layer "F.Cu") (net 2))
 (segment (start 153.0605 94.996) (end 153.0605 96.52) (width 0.508) (layer "F.Cu") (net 2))
 (segment (start 153.0605 94.996) (end 153.0605 94.3865) (width 0.508) (layer "F.Cu") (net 2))
 (segment (start 153.0605 96.52) (end 153.0605 98.1685) (width 0.508) (layer "F.Cu") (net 2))
 (segment (start 145.796 93.599) (end 145.034 94.361) (width 0.508) (layer "F.Cu") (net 2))
 (segment (start 152.273 93.599) (end 145.796 93.599) (width 0.508) (layer "F.Cu") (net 2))
 (segment (start 151.4855 96.52) (end 150.0125 96.52) (width 0.508) (layer "F.Cu") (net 5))
 (segment (start 150.0125 96.52) (end 149.987 96.5455) (width 0.508) (layer "F.Cu") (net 5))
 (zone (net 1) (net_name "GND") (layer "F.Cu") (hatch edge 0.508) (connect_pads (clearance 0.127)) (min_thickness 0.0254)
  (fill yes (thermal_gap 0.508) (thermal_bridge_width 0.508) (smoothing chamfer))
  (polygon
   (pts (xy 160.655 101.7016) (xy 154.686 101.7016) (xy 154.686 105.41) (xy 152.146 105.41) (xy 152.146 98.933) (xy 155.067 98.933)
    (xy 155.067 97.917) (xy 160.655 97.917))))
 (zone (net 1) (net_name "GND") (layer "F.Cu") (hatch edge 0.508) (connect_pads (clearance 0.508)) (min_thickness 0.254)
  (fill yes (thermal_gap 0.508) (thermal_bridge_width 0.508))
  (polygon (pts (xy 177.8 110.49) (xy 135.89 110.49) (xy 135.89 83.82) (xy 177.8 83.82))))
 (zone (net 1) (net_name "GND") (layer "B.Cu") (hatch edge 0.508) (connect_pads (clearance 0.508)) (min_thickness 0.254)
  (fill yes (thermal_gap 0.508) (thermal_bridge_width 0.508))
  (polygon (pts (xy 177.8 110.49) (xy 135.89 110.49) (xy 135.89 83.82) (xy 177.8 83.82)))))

